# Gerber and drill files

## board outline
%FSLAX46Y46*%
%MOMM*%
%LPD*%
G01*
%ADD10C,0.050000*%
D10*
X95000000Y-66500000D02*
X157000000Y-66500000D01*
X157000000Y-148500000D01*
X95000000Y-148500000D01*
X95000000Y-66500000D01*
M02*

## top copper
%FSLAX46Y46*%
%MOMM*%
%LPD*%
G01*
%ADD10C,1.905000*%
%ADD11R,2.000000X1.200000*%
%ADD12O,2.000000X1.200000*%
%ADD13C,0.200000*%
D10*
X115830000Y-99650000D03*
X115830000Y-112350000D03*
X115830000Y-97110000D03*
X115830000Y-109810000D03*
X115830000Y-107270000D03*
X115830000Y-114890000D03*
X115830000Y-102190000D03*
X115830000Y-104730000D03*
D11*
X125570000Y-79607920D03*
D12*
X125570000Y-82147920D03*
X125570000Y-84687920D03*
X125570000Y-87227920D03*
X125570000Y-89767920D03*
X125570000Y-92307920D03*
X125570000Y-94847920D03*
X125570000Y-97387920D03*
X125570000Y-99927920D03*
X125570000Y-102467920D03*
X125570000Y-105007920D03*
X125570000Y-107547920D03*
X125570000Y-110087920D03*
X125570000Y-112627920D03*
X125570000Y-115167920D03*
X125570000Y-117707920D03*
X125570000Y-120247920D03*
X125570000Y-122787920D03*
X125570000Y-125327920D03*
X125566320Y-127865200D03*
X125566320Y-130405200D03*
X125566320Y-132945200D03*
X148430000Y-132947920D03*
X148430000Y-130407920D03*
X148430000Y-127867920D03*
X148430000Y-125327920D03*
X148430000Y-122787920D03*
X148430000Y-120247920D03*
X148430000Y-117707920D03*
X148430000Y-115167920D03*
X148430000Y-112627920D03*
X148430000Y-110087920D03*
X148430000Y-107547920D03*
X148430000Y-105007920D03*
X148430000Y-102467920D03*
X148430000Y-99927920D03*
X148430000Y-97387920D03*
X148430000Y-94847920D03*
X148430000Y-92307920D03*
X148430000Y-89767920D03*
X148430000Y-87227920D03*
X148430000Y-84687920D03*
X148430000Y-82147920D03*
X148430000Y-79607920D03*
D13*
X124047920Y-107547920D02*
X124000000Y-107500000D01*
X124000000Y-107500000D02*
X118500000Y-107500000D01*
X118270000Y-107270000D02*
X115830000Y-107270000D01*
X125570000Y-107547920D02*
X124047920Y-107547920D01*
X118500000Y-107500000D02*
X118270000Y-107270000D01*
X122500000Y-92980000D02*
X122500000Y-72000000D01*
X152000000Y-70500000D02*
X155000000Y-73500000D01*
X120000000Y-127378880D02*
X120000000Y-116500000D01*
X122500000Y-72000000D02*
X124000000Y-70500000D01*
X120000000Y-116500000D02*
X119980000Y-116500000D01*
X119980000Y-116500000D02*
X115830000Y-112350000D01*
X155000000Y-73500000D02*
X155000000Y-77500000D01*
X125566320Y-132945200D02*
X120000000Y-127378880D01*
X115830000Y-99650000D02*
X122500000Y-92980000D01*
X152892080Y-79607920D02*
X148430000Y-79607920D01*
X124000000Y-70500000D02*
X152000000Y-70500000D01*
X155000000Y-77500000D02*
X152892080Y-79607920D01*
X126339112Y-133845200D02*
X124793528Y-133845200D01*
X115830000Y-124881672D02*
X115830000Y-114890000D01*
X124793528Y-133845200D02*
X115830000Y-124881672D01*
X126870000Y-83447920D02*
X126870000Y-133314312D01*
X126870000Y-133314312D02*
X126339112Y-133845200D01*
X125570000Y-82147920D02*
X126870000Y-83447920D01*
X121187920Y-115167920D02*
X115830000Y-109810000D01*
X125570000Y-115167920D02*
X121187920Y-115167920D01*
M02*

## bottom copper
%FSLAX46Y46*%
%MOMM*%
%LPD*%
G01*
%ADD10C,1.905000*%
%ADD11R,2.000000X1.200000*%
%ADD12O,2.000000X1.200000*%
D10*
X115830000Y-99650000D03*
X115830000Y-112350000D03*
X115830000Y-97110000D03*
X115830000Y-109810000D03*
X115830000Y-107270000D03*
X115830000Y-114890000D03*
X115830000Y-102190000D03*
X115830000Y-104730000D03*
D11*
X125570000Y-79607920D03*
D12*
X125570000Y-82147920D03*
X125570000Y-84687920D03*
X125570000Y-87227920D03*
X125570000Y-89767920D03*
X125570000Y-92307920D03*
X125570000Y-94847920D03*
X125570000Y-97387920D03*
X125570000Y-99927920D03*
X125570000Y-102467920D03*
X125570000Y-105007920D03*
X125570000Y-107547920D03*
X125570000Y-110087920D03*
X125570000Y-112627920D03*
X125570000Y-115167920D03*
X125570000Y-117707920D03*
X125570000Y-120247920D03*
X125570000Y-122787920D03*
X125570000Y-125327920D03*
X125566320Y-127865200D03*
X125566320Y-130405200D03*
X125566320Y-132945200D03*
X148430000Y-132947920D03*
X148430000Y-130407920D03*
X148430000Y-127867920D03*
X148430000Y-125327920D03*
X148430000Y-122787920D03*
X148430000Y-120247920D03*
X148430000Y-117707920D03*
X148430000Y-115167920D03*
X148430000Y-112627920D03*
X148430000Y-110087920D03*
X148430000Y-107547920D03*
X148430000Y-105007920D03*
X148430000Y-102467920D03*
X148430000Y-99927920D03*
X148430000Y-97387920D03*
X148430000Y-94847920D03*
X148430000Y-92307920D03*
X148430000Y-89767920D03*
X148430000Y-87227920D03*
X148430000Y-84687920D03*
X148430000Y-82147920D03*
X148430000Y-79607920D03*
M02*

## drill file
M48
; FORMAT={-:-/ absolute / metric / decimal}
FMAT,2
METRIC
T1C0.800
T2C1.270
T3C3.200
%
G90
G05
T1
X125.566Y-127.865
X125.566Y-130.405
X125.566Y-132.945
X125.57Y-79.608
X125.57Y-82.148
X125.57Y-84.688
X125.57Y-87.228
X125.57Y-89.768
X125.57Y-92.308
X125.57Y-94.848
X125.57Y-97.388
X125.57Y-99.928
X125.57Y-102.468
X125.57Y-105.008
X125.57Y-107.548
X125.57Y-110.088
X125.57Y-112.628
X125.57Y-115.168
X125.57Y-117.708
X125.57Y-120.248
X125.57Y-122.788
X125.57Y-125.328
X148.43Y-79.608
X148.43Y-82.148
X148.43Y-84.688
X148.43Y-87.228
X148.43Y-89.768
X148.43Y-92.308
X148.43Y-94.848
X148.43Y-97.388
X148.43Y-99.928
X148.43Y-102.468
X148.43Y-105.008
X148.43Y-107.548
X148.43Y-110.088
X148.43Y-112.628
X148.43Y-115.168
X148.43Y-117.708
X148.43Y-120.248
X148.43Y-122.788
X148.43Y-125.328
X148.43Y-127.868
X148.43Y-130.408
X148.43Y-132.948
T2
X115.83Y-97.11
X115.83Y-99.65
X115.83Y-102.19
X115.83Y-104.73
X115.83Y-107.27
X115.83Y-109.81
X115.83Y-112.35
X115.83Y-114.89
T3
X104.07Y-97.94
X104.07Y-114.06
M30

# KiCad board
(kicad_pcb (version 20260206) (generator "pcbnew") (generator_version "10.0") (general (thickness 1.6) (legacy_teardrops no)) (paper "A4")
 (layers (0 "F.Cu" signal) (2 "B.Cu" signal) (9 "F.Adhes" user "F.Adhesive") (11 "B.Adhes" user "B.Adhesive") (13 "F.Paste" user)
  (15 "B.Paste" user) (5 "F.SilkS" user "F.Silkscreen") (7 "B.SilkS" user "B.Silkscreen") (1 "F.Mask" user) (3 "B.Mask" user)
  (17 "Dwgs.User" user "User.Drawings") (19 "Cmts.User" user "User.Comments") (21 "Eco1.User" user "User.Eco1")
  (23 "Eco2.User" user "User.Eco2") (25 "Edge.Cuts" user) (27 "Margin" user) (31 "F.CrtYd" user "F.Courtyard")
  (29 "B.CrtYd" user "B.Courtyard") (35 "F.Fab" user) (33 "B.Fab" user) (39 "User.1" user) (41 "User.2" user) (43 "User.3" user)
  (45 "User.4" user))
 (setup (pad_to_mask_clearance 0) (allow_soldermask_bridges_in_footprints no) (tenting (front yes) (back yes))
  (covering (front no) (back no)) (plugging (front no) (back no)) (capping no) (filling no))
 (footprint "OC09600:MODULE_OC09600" (layer "F.Cu") (at 109.5 106 180)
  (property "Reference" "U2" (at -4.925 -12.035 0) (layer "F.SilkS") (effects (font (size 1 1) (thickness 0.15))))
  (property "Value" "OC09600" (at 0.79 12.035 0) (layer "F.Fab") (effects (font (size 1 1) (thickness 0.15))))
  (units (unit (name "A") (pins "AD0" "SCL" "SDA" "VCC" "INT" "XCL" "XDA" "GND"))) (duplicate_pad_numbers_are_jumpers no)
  (pad "" np_thru_hole circle (at 5.43 -8.06 180) (size 3.2 3.2) (drill 3.2) (layers "*.Cu" "*.Mask"))
  (pad "" np_thru_hole circle (at 5.43 8.06 180) (size 3.2 3.2) (drill 3.2) (layers "*.Cu" "*.Mask"))
  (pad "AD0" thru_hole circle (at -6.33 6.35 180) (size 1.905 1.905) (drill 1.27) (layers "*.Cu" "*.Mask") (remove_unused_layers no)
   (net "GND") (solder_mask_margin 0.102))
  (pad "GND" thru_hole circle (at -6.33 -6.35 180) (size 1.905 1.905) (drill 1.27) (layers "*.Cu" "*.Mask") (remove_unused_layers no)
   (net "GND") (solder_mask_margin 0.102))
  (pad "INT" thru_hole circle (at -6.33 8.89 180) (size 1.905 1.905) (drill 1.27) (layers "*.Cu" "*.Mask") (remove_unused_layers no)
   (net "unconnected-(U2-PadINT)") (solder_mask_margin 0.102))
  (pad "SCL" thru_hole circle (at -6.33 -3.81 180) (size 1.905 1.905) (drill 1.27) (layers "*.Cu" "*.Mask") (remove_unused_layers no)
   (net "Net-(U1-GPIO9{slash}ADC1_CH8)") (solder_mask_margin 0.102))
  (pad "SDA" thru_hole circle (at -6.33 -1.27 180) (size 1.905 1.905) (drill 1.27) (layers "*.Cu" "*.Mask") (remove_unused_layers no)
   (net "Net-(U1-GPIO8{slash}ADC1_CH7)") (solder_mask_margin 0.102))
  (pad "VCC" thru_hole circle (at -6.33 -8.89 180) (size 1.905 1.905) (drill 1.27) (layers "*.Cu" "*.Mask") (remove_unused_layers no)
   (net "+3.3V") (solder_mask_margin 0.102))
  (pad "XCL" thru_hole circle (at -6.33 3.81 180) (size 1.905 1.905) (drill 1.27) (layers "*.Cu" "*.Mask") (remove_unused_layers no)
   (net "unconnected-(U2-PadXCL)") (solder_mask_margin 0.102))
  (pad "XDA" thru_hole circle (at -6.33 1.27 180) (size 1.905 1.905) (drill 1.27) (layers "*.Cu" "*.Mask") (remove_unused_layers no)
   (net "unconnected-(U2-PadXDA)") (solder_mask_margin 0.102)))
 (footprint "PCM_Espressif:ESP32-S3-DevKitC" (layer "F.Cu") (at 125.57 79.60792)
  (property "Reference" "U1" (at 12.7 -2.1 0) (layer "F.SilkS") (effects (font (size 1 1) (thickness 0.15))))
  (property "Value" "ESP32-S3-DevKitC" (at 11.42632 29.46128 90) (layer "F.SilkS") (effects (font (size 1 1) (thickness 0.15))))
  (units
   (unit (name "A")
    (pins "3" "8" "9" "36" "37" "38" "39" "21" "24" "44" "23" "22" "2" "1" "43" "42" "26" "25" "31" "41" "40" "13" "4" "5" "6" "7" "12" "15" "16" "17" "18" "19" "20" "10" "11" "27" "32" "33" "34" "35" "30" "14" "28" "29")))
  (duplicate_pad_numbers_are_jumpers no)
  (pad "1" thru_hole rect (at 0 0 270) (size 1.2 2) (drill 0.8) (layers "*.Cu" "*.Mask") (remove_unused_layers no) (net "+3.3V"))
  (pad "2" thru_hole oval (at 0 2.54 270) (size 1.2 2) (drill 0.8) (layers "*.Cu" "*.Mask") (remove_unused_layers no) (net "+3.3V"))
  (pad "3" thru_hole oval (at 0 5.08 270) (size 1.2 2) (drill 0.8) (layers "*.Cu" "*.Mask") (remove_unused_layers no)
   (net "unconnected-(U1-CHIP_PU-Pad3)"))
  (pad "4" thru_hole oval (at 0 7.62 270) (size 1.2 2) (drill 0.8) (layers "*.Cu" "*.Mask") (remove_unused_layers no)
   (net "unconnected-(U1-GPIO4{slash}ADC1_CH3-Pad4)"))
  (pad "5" thru_hole oval (at 0 10.16 270) (size 1.2 2) (drill 0.8) (layers "*.Cu" "*.Mask") (remove_unused_layers no)
   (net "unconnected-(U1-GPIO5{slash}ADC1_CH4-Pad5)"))
  (pad "6" thru_hole oval (at 0 12.7 270) (size 1.2 2) (drill 0.8) (layers "*.Cu" "*.Mask") (remove_unused_layers no)
   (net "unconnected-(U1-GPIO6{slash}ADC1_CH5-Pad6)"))
  (pad "7" thru_hole oval (at 0 15.24 270) (size 1.2 2) (drill 0.8) (layers "*.Cu" "*.Mask") (remove_unused_layers no)
   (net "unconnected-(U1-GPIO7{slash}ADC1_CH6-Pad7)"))
  (pad "8" thru_hole oval (at 0 17.78 270) (size 1.2 2) (drill 0.8) (layers "*.Cu" "*.Mask") (remove_unused_layers no)
   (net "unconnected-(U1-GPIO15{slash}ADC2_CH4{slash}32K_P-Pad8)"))
  (pad "9" thru_hole oval (at 0 20.32 270) (size 1.2 2) (drill 0.8) (layers "*.Cu" "*.Mask") (remove_unused_layers no)
   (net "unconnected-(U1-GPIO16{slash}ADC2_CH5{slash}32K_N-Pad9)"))
  (pad "10" thru_hole oval (at 0 22.86 270) (size 1.2 2) (drill 0.8) (layers "*.Cu" "*.Mask") (remove_unused_layers no)
   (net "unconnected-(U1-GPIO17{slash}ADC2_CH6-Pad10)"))
  (pad "11" thru_hole oval (at 0 25.4 270) (size 1.2 2) (drill 0.8) (layers "*.Cu" "*.Mask") (remove_unused_layers no)
   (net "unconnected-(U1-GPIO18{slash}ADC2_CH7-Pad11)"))
  (pad "12" thru_hole oval (at 0 27.94 270) (size 1.2 2) (drill 0.8) (layers "*.Cu" "*.Mask") (remove_unused_layers no)
   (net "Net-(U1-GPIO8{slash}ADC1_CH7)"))
  (pad "13" thru_hole oval (at 0 30.48 270) (size 1.2 2) (drill 0.8) (layers "*.Cu" "*.Mask") (remove_unused_layers no)
   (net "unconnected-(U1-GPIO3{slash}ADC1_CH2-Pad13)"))
  (pad "14" thru_hole oval (at 0 33.02 270) (size 1.2 2) (drill 0.8) (layers "*.Cu" "*.Mask") (remove_unused_layers no)
   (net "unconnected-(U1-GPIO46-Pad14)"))
  (pad "15" thru_hole oval (at 0 35.56 270) (size 1.2 2) (drill 0.8) (layers "*.Cu" "*.Mask") (remove_unused_layers no)
   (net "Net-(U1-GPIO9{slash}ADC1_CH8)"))
  (pad "16" thru_hole oval (at 0 38.1 270) (size 1.2 2) (drill 0.8) (layers "*.Cu" "*.Mask") (remove_unused_layers no)
   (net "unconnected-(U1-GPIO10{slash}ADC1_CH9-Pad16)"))
  (pad "17" thru_hole oval (at 0 40.64 270) (size 1.2 2) (drill 0.8) (layers "*.Cu" "*.Mask") (remove_unused_layers no)
   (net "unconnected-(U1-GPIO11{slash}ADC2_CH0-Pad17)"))
  (pad "18" thru_hole oval (at 0 43.18 270) (size 1.2 2) (drill 0.8) (layers "*.Cu" "*.Mask") (remove_unused_layers no)
   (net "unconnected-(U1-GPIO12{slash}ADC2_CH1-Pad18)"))
  (pad "19" thru_hole oval (at 0 45.72 270) (size 1.2 2) (drill 0.8) (layers "*.Cu" "*.Mask") (remove_unused_layers no)
   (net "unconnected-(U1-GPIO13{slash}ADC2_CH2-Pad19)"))
  (pad "20" thru_hole oval (at -0.00368 48.25728 270) (size 1.2 2) (drill 0.8) (layers "*.Cu" "*.Mask") (remove_unused_layers no)
   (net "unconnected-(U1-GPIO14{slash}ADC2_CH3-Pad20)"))
  (pad "21" thru_hole oval (at -0.00368 50.79728 270) (size 1.2 2) (drill 0.8) (layers "*.Cu" "*.Mask") (remove_unused_layers no)
   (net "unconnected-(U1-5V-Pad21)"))
  (pad "22" thru_hole oval (at -0.00368 53.33728 270) (size 1.2 2) (drill 0.8) (layers "*.Cu" "*.Mask") (remove_unused_layers no)
   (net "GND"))
  (pad "23" thru_hole oval (at 22.86 53.34 270) (size 1.2 2) (drill 0.8) (layers "*.Cu" "*.Mask") (remove_unused_layers no) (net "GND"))
  (pad "24" thru_hole oval (at 22.86 50.8 270) (size 1.2 2) (drill 0.8) (layers "*.Cu" "*.Mask") (remove_unused_layers no) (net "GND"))
  (pad "25" thru_hole oval (at 22.86 48.26 270) (size 1.2 2) (drill 0.8) (layers "*.Cu" "*.Mask") (remove_unused_layers no)
   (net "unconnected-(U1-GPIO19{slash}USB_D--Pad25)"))
  (pad "26" thru_hole oval (at 22.86 45.72 270) (size 1.2 2) (drill 0.8) (layers "*.Cu" "*.Mask") (remove_unused_layers no)
   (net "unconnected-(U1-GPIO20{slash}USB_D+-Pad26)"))
  (pad "27" thru_hole oval (at 22.86 43.18 270) (size 1.2 2) (drill 0.8) (layers "*.Cu" "*.Mask") (remove_unused_layers no)
   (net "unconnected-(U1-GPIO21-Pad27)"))
  (pad "28" thru_hole oval (at 22.86 40.64 270) (size 1.2 2) (drill 0.8) (layers "*.Cu" "*.Mask") (remove_unused_layers no)
   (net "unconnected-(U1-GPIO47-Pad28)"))
  (pad "29" thru_hole oval (at 22.86 38.1 270) (size 1.2 2) (drill 0.8) (layers "*.Cu" "*.Mask") (remove_unused_layers no)
   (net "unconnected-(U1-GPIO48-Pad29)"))
  (pad "30" thru_hole oval (at 22.86 35.56 270) (size 1.2 2) (drill 0.8) (layers "*.Cu" "*.Mask") (remove_unused_layers no)
   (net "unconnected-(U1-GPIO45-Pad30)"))
  (pad "31" thru_hole oval (at 22.86 33.02 270) (size 1.2 2) (drill 0.8) (layers "*.Cu" "*.Mask") (remove_unused_layers no)
   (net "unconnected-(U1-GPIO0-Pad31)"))
  (pad "32" thru_hole oval (at 22.86 30.48 270) (size 1.2 2) (drill 0.8) (layers "*.Cu" "*.Mask") (remove_unused_layers no)
   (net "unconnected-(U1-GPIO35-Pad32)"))
  (pad "33" thru_hole oval (at 22.86 27.94 270) (size 1.2 2) (drill 0.8) (layers "*.Cu" "*.Mask") (remove_unused_layers no)
   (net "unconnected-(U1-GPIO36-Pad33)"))
  (pad "34" thru_hole oval (at 22.86 25.4 270) (size 1.2 2) (drill 0.8) (layers "*.Cu" "*.Mask") (remove_unused_layers no)
   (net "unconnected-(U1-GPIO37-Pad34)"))
  (pad "35" thru_hole oval (at 22.86 22.86 270) (size 1.2 2) (drill 0.8) (layers "*.Cu" "*.Mask") (remove_unused_layers no)
   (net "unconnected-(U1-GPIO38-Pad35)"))
  (pad "36" thru_hole oval (at 22.86 20.32 270) (size 1.2 2) (drill 0.8) (layers "*.Cu" "*.Mask") (remove_unused_layers no)
   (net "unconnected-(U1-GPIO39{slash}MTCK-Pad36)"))
  (pad "37" thru_hole oval (at 22.86 17.78 270) (size 1.2 2) (drill 0.8) (layers "*.Cu" "*.Mask") (remove_unused_layers no)
   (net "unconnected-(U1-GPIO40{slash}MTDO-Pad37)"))
  (pad "38" thru_hole oval (at 22.86 15.24 270) (size 1.2 2) (drill 0.8) (layers "*.Cu" "*.Mask") (remove_unused_layers no)
   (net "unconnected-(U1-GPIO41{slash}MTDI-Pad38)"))
  (pad "39" thru_hole oval (at 22.86 12.7 270) (size 1.2 2) (drill 0.8) (layers "*.Cu" "*.Mask") (remove_unused_layers no)
   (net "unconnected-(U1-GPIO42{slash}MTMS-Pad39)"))
  (pad "40" thru_hole oval (at 22.86 10.16 270) (size 1.2 2) (drill 0.8) (layers "*.Cu" "*.Mask") (remove_unused_layers no)
   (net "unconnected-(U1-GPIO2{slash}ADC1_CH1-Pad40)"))
  (pad "41" thru_hole oval (at 22.86 7.62 270) (size 1.2 2) (drill 0.8) (layers "*.Cu" "*.Mask") (remove_unused_layers no)
   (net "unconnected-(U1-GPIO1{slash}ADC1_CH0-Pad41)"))
  (pad "42" thru_hole oval (at 22.86 5.08 270) (size 1.2 2) (drill 0.8) (layers "*.Cu" "*.Mask") (remove_unused_layers no)
   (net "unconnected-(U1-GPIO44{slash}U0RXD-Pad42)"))
  (pad "43" thru_hole oval (at 22.86 2.54 270) (size 1.2 2) (drill 0.8) (layers "*.Cu" "*.Mask") (remove_unused_layers no)
   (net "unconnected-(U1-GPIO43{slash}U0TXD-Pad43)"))
  (pad "44" thru_hole oval (at 22.86 0 270) (size 1.2 2) (drill 0.8) (layers "*.Cu" "*.Mask") (remove_unused_layers no) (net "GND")))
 (gr_rect (start 95 66.5) (end 157 148.5) (stroke (width 0.05) (type default)) (fill no) (layer "Edge.Cuts"))
 (segment (start 124.04792 107.54792) (end 124 107.5) (width 0.2) (layer "F.Cu") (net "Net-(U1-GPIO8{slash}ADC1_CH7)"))
 (segment (start 124 107.5) (end 118.5 107.5) (width 0.2) (layer "F.Cu") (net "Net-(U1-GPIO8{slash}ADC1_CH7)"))
 (segment (start 118.27 107.27) (end 115.83 107.27) (width 0.2) (layer "F.Cu") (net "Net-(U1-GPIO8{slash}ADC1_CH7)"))
 (segment (start 125.57 107.54792) (end 124.04792 107.54792) (width 0.2) (layer "F.Cu") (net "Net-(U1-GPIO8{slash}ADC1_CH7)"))
 (segment (start 118.5 107.5) (end 118.27 107.27) (width 0.2) (layer "F.Cu") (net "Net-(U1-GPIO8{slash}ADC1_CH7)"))
 (segment (start 122.5 92.98) (end 122.5 72) (width 0.2) (layer "F.Cu") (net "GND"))
 (segment (start 152 70.5) (end 155 73.5) (width 0.2) (layer "F.Cu") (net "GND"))
 (segment (start 120 127.37888) (end 120 116.5) (width 0.2) (layer "F.Cu") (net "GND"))
 (segment (start 122.5 72) (end 124 70.5) (width 0.2) (layer "F.Cu") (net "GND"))
 (segment (start 120 116.5) (end 119.98 116.5) (width 0.2) (layer "F.Cu") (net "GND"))
 (segment (start 119.98 116.5) (end 115.83 112.35) (width 0.2) (layer "F.Cu") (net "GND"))
 (segment (start 155 73.5) (end 155 77.5) (width 0.2) (layer "F.Cu") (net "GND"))
 (segment (start 125.56632 132.9452) (end 120 127.37888) (width 0.2) (layer "F.Cu") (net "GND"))
 (segment (start 115.83 99.65) (end 122.5 92.98) (width 0.2) (layer "F.Cu") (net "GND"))
 (segment (start 152.89208 79.60792) (end 148.43 79.60792) (width 0.2) (layer "F.Cu") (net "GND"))
 (segment (start 124 70.5) (end 152 70.5) (width 0.2) (layer "F.Cu") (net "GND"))
 (segment (start 155 77.5) (end 152.89208 79.60792) (width 0.2) (layer "F.Cu") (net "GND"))
 (segment (start 126.339112 133.8452) (end 124.793528 133.8452) (width 0.2) (layer "F.Cu") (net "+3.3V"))
 (segment (start 115.83 124.881672) (end 115.83 114.89) (width 0.2) (layer "F.Cu") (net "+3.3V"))
 (segment (start 124.793528 133.8452) (end 115.83 124.881672) (width 0.2) (layer "F.Cu") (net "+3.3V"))
 (segment (start 126.87 83.44792) (end 126.87 133.314312) (width 0.2) (layer "F.Cu") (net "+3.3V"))
 (segment (start 126.87 133.314312) (end 126.339112 133.8452) (width 0.2) (layer "F.Cu") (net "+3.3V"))
 (segment (start 125.57 82.14792) (end 126.87 83.44792) (width 0.2) (layer "F.Cu") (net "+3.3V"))
 (segment (start 121.18792 115.16792) (end 115.83 109.81) (width 0.2) (layer "F.Cu") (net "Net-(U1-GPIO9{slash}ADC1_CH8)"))
 (segment (start 125.57 115.16792) (end 121.18792 115.16792) (width 0.2) (layer "F.Cu") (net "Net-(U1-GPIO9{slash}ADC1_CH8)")))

